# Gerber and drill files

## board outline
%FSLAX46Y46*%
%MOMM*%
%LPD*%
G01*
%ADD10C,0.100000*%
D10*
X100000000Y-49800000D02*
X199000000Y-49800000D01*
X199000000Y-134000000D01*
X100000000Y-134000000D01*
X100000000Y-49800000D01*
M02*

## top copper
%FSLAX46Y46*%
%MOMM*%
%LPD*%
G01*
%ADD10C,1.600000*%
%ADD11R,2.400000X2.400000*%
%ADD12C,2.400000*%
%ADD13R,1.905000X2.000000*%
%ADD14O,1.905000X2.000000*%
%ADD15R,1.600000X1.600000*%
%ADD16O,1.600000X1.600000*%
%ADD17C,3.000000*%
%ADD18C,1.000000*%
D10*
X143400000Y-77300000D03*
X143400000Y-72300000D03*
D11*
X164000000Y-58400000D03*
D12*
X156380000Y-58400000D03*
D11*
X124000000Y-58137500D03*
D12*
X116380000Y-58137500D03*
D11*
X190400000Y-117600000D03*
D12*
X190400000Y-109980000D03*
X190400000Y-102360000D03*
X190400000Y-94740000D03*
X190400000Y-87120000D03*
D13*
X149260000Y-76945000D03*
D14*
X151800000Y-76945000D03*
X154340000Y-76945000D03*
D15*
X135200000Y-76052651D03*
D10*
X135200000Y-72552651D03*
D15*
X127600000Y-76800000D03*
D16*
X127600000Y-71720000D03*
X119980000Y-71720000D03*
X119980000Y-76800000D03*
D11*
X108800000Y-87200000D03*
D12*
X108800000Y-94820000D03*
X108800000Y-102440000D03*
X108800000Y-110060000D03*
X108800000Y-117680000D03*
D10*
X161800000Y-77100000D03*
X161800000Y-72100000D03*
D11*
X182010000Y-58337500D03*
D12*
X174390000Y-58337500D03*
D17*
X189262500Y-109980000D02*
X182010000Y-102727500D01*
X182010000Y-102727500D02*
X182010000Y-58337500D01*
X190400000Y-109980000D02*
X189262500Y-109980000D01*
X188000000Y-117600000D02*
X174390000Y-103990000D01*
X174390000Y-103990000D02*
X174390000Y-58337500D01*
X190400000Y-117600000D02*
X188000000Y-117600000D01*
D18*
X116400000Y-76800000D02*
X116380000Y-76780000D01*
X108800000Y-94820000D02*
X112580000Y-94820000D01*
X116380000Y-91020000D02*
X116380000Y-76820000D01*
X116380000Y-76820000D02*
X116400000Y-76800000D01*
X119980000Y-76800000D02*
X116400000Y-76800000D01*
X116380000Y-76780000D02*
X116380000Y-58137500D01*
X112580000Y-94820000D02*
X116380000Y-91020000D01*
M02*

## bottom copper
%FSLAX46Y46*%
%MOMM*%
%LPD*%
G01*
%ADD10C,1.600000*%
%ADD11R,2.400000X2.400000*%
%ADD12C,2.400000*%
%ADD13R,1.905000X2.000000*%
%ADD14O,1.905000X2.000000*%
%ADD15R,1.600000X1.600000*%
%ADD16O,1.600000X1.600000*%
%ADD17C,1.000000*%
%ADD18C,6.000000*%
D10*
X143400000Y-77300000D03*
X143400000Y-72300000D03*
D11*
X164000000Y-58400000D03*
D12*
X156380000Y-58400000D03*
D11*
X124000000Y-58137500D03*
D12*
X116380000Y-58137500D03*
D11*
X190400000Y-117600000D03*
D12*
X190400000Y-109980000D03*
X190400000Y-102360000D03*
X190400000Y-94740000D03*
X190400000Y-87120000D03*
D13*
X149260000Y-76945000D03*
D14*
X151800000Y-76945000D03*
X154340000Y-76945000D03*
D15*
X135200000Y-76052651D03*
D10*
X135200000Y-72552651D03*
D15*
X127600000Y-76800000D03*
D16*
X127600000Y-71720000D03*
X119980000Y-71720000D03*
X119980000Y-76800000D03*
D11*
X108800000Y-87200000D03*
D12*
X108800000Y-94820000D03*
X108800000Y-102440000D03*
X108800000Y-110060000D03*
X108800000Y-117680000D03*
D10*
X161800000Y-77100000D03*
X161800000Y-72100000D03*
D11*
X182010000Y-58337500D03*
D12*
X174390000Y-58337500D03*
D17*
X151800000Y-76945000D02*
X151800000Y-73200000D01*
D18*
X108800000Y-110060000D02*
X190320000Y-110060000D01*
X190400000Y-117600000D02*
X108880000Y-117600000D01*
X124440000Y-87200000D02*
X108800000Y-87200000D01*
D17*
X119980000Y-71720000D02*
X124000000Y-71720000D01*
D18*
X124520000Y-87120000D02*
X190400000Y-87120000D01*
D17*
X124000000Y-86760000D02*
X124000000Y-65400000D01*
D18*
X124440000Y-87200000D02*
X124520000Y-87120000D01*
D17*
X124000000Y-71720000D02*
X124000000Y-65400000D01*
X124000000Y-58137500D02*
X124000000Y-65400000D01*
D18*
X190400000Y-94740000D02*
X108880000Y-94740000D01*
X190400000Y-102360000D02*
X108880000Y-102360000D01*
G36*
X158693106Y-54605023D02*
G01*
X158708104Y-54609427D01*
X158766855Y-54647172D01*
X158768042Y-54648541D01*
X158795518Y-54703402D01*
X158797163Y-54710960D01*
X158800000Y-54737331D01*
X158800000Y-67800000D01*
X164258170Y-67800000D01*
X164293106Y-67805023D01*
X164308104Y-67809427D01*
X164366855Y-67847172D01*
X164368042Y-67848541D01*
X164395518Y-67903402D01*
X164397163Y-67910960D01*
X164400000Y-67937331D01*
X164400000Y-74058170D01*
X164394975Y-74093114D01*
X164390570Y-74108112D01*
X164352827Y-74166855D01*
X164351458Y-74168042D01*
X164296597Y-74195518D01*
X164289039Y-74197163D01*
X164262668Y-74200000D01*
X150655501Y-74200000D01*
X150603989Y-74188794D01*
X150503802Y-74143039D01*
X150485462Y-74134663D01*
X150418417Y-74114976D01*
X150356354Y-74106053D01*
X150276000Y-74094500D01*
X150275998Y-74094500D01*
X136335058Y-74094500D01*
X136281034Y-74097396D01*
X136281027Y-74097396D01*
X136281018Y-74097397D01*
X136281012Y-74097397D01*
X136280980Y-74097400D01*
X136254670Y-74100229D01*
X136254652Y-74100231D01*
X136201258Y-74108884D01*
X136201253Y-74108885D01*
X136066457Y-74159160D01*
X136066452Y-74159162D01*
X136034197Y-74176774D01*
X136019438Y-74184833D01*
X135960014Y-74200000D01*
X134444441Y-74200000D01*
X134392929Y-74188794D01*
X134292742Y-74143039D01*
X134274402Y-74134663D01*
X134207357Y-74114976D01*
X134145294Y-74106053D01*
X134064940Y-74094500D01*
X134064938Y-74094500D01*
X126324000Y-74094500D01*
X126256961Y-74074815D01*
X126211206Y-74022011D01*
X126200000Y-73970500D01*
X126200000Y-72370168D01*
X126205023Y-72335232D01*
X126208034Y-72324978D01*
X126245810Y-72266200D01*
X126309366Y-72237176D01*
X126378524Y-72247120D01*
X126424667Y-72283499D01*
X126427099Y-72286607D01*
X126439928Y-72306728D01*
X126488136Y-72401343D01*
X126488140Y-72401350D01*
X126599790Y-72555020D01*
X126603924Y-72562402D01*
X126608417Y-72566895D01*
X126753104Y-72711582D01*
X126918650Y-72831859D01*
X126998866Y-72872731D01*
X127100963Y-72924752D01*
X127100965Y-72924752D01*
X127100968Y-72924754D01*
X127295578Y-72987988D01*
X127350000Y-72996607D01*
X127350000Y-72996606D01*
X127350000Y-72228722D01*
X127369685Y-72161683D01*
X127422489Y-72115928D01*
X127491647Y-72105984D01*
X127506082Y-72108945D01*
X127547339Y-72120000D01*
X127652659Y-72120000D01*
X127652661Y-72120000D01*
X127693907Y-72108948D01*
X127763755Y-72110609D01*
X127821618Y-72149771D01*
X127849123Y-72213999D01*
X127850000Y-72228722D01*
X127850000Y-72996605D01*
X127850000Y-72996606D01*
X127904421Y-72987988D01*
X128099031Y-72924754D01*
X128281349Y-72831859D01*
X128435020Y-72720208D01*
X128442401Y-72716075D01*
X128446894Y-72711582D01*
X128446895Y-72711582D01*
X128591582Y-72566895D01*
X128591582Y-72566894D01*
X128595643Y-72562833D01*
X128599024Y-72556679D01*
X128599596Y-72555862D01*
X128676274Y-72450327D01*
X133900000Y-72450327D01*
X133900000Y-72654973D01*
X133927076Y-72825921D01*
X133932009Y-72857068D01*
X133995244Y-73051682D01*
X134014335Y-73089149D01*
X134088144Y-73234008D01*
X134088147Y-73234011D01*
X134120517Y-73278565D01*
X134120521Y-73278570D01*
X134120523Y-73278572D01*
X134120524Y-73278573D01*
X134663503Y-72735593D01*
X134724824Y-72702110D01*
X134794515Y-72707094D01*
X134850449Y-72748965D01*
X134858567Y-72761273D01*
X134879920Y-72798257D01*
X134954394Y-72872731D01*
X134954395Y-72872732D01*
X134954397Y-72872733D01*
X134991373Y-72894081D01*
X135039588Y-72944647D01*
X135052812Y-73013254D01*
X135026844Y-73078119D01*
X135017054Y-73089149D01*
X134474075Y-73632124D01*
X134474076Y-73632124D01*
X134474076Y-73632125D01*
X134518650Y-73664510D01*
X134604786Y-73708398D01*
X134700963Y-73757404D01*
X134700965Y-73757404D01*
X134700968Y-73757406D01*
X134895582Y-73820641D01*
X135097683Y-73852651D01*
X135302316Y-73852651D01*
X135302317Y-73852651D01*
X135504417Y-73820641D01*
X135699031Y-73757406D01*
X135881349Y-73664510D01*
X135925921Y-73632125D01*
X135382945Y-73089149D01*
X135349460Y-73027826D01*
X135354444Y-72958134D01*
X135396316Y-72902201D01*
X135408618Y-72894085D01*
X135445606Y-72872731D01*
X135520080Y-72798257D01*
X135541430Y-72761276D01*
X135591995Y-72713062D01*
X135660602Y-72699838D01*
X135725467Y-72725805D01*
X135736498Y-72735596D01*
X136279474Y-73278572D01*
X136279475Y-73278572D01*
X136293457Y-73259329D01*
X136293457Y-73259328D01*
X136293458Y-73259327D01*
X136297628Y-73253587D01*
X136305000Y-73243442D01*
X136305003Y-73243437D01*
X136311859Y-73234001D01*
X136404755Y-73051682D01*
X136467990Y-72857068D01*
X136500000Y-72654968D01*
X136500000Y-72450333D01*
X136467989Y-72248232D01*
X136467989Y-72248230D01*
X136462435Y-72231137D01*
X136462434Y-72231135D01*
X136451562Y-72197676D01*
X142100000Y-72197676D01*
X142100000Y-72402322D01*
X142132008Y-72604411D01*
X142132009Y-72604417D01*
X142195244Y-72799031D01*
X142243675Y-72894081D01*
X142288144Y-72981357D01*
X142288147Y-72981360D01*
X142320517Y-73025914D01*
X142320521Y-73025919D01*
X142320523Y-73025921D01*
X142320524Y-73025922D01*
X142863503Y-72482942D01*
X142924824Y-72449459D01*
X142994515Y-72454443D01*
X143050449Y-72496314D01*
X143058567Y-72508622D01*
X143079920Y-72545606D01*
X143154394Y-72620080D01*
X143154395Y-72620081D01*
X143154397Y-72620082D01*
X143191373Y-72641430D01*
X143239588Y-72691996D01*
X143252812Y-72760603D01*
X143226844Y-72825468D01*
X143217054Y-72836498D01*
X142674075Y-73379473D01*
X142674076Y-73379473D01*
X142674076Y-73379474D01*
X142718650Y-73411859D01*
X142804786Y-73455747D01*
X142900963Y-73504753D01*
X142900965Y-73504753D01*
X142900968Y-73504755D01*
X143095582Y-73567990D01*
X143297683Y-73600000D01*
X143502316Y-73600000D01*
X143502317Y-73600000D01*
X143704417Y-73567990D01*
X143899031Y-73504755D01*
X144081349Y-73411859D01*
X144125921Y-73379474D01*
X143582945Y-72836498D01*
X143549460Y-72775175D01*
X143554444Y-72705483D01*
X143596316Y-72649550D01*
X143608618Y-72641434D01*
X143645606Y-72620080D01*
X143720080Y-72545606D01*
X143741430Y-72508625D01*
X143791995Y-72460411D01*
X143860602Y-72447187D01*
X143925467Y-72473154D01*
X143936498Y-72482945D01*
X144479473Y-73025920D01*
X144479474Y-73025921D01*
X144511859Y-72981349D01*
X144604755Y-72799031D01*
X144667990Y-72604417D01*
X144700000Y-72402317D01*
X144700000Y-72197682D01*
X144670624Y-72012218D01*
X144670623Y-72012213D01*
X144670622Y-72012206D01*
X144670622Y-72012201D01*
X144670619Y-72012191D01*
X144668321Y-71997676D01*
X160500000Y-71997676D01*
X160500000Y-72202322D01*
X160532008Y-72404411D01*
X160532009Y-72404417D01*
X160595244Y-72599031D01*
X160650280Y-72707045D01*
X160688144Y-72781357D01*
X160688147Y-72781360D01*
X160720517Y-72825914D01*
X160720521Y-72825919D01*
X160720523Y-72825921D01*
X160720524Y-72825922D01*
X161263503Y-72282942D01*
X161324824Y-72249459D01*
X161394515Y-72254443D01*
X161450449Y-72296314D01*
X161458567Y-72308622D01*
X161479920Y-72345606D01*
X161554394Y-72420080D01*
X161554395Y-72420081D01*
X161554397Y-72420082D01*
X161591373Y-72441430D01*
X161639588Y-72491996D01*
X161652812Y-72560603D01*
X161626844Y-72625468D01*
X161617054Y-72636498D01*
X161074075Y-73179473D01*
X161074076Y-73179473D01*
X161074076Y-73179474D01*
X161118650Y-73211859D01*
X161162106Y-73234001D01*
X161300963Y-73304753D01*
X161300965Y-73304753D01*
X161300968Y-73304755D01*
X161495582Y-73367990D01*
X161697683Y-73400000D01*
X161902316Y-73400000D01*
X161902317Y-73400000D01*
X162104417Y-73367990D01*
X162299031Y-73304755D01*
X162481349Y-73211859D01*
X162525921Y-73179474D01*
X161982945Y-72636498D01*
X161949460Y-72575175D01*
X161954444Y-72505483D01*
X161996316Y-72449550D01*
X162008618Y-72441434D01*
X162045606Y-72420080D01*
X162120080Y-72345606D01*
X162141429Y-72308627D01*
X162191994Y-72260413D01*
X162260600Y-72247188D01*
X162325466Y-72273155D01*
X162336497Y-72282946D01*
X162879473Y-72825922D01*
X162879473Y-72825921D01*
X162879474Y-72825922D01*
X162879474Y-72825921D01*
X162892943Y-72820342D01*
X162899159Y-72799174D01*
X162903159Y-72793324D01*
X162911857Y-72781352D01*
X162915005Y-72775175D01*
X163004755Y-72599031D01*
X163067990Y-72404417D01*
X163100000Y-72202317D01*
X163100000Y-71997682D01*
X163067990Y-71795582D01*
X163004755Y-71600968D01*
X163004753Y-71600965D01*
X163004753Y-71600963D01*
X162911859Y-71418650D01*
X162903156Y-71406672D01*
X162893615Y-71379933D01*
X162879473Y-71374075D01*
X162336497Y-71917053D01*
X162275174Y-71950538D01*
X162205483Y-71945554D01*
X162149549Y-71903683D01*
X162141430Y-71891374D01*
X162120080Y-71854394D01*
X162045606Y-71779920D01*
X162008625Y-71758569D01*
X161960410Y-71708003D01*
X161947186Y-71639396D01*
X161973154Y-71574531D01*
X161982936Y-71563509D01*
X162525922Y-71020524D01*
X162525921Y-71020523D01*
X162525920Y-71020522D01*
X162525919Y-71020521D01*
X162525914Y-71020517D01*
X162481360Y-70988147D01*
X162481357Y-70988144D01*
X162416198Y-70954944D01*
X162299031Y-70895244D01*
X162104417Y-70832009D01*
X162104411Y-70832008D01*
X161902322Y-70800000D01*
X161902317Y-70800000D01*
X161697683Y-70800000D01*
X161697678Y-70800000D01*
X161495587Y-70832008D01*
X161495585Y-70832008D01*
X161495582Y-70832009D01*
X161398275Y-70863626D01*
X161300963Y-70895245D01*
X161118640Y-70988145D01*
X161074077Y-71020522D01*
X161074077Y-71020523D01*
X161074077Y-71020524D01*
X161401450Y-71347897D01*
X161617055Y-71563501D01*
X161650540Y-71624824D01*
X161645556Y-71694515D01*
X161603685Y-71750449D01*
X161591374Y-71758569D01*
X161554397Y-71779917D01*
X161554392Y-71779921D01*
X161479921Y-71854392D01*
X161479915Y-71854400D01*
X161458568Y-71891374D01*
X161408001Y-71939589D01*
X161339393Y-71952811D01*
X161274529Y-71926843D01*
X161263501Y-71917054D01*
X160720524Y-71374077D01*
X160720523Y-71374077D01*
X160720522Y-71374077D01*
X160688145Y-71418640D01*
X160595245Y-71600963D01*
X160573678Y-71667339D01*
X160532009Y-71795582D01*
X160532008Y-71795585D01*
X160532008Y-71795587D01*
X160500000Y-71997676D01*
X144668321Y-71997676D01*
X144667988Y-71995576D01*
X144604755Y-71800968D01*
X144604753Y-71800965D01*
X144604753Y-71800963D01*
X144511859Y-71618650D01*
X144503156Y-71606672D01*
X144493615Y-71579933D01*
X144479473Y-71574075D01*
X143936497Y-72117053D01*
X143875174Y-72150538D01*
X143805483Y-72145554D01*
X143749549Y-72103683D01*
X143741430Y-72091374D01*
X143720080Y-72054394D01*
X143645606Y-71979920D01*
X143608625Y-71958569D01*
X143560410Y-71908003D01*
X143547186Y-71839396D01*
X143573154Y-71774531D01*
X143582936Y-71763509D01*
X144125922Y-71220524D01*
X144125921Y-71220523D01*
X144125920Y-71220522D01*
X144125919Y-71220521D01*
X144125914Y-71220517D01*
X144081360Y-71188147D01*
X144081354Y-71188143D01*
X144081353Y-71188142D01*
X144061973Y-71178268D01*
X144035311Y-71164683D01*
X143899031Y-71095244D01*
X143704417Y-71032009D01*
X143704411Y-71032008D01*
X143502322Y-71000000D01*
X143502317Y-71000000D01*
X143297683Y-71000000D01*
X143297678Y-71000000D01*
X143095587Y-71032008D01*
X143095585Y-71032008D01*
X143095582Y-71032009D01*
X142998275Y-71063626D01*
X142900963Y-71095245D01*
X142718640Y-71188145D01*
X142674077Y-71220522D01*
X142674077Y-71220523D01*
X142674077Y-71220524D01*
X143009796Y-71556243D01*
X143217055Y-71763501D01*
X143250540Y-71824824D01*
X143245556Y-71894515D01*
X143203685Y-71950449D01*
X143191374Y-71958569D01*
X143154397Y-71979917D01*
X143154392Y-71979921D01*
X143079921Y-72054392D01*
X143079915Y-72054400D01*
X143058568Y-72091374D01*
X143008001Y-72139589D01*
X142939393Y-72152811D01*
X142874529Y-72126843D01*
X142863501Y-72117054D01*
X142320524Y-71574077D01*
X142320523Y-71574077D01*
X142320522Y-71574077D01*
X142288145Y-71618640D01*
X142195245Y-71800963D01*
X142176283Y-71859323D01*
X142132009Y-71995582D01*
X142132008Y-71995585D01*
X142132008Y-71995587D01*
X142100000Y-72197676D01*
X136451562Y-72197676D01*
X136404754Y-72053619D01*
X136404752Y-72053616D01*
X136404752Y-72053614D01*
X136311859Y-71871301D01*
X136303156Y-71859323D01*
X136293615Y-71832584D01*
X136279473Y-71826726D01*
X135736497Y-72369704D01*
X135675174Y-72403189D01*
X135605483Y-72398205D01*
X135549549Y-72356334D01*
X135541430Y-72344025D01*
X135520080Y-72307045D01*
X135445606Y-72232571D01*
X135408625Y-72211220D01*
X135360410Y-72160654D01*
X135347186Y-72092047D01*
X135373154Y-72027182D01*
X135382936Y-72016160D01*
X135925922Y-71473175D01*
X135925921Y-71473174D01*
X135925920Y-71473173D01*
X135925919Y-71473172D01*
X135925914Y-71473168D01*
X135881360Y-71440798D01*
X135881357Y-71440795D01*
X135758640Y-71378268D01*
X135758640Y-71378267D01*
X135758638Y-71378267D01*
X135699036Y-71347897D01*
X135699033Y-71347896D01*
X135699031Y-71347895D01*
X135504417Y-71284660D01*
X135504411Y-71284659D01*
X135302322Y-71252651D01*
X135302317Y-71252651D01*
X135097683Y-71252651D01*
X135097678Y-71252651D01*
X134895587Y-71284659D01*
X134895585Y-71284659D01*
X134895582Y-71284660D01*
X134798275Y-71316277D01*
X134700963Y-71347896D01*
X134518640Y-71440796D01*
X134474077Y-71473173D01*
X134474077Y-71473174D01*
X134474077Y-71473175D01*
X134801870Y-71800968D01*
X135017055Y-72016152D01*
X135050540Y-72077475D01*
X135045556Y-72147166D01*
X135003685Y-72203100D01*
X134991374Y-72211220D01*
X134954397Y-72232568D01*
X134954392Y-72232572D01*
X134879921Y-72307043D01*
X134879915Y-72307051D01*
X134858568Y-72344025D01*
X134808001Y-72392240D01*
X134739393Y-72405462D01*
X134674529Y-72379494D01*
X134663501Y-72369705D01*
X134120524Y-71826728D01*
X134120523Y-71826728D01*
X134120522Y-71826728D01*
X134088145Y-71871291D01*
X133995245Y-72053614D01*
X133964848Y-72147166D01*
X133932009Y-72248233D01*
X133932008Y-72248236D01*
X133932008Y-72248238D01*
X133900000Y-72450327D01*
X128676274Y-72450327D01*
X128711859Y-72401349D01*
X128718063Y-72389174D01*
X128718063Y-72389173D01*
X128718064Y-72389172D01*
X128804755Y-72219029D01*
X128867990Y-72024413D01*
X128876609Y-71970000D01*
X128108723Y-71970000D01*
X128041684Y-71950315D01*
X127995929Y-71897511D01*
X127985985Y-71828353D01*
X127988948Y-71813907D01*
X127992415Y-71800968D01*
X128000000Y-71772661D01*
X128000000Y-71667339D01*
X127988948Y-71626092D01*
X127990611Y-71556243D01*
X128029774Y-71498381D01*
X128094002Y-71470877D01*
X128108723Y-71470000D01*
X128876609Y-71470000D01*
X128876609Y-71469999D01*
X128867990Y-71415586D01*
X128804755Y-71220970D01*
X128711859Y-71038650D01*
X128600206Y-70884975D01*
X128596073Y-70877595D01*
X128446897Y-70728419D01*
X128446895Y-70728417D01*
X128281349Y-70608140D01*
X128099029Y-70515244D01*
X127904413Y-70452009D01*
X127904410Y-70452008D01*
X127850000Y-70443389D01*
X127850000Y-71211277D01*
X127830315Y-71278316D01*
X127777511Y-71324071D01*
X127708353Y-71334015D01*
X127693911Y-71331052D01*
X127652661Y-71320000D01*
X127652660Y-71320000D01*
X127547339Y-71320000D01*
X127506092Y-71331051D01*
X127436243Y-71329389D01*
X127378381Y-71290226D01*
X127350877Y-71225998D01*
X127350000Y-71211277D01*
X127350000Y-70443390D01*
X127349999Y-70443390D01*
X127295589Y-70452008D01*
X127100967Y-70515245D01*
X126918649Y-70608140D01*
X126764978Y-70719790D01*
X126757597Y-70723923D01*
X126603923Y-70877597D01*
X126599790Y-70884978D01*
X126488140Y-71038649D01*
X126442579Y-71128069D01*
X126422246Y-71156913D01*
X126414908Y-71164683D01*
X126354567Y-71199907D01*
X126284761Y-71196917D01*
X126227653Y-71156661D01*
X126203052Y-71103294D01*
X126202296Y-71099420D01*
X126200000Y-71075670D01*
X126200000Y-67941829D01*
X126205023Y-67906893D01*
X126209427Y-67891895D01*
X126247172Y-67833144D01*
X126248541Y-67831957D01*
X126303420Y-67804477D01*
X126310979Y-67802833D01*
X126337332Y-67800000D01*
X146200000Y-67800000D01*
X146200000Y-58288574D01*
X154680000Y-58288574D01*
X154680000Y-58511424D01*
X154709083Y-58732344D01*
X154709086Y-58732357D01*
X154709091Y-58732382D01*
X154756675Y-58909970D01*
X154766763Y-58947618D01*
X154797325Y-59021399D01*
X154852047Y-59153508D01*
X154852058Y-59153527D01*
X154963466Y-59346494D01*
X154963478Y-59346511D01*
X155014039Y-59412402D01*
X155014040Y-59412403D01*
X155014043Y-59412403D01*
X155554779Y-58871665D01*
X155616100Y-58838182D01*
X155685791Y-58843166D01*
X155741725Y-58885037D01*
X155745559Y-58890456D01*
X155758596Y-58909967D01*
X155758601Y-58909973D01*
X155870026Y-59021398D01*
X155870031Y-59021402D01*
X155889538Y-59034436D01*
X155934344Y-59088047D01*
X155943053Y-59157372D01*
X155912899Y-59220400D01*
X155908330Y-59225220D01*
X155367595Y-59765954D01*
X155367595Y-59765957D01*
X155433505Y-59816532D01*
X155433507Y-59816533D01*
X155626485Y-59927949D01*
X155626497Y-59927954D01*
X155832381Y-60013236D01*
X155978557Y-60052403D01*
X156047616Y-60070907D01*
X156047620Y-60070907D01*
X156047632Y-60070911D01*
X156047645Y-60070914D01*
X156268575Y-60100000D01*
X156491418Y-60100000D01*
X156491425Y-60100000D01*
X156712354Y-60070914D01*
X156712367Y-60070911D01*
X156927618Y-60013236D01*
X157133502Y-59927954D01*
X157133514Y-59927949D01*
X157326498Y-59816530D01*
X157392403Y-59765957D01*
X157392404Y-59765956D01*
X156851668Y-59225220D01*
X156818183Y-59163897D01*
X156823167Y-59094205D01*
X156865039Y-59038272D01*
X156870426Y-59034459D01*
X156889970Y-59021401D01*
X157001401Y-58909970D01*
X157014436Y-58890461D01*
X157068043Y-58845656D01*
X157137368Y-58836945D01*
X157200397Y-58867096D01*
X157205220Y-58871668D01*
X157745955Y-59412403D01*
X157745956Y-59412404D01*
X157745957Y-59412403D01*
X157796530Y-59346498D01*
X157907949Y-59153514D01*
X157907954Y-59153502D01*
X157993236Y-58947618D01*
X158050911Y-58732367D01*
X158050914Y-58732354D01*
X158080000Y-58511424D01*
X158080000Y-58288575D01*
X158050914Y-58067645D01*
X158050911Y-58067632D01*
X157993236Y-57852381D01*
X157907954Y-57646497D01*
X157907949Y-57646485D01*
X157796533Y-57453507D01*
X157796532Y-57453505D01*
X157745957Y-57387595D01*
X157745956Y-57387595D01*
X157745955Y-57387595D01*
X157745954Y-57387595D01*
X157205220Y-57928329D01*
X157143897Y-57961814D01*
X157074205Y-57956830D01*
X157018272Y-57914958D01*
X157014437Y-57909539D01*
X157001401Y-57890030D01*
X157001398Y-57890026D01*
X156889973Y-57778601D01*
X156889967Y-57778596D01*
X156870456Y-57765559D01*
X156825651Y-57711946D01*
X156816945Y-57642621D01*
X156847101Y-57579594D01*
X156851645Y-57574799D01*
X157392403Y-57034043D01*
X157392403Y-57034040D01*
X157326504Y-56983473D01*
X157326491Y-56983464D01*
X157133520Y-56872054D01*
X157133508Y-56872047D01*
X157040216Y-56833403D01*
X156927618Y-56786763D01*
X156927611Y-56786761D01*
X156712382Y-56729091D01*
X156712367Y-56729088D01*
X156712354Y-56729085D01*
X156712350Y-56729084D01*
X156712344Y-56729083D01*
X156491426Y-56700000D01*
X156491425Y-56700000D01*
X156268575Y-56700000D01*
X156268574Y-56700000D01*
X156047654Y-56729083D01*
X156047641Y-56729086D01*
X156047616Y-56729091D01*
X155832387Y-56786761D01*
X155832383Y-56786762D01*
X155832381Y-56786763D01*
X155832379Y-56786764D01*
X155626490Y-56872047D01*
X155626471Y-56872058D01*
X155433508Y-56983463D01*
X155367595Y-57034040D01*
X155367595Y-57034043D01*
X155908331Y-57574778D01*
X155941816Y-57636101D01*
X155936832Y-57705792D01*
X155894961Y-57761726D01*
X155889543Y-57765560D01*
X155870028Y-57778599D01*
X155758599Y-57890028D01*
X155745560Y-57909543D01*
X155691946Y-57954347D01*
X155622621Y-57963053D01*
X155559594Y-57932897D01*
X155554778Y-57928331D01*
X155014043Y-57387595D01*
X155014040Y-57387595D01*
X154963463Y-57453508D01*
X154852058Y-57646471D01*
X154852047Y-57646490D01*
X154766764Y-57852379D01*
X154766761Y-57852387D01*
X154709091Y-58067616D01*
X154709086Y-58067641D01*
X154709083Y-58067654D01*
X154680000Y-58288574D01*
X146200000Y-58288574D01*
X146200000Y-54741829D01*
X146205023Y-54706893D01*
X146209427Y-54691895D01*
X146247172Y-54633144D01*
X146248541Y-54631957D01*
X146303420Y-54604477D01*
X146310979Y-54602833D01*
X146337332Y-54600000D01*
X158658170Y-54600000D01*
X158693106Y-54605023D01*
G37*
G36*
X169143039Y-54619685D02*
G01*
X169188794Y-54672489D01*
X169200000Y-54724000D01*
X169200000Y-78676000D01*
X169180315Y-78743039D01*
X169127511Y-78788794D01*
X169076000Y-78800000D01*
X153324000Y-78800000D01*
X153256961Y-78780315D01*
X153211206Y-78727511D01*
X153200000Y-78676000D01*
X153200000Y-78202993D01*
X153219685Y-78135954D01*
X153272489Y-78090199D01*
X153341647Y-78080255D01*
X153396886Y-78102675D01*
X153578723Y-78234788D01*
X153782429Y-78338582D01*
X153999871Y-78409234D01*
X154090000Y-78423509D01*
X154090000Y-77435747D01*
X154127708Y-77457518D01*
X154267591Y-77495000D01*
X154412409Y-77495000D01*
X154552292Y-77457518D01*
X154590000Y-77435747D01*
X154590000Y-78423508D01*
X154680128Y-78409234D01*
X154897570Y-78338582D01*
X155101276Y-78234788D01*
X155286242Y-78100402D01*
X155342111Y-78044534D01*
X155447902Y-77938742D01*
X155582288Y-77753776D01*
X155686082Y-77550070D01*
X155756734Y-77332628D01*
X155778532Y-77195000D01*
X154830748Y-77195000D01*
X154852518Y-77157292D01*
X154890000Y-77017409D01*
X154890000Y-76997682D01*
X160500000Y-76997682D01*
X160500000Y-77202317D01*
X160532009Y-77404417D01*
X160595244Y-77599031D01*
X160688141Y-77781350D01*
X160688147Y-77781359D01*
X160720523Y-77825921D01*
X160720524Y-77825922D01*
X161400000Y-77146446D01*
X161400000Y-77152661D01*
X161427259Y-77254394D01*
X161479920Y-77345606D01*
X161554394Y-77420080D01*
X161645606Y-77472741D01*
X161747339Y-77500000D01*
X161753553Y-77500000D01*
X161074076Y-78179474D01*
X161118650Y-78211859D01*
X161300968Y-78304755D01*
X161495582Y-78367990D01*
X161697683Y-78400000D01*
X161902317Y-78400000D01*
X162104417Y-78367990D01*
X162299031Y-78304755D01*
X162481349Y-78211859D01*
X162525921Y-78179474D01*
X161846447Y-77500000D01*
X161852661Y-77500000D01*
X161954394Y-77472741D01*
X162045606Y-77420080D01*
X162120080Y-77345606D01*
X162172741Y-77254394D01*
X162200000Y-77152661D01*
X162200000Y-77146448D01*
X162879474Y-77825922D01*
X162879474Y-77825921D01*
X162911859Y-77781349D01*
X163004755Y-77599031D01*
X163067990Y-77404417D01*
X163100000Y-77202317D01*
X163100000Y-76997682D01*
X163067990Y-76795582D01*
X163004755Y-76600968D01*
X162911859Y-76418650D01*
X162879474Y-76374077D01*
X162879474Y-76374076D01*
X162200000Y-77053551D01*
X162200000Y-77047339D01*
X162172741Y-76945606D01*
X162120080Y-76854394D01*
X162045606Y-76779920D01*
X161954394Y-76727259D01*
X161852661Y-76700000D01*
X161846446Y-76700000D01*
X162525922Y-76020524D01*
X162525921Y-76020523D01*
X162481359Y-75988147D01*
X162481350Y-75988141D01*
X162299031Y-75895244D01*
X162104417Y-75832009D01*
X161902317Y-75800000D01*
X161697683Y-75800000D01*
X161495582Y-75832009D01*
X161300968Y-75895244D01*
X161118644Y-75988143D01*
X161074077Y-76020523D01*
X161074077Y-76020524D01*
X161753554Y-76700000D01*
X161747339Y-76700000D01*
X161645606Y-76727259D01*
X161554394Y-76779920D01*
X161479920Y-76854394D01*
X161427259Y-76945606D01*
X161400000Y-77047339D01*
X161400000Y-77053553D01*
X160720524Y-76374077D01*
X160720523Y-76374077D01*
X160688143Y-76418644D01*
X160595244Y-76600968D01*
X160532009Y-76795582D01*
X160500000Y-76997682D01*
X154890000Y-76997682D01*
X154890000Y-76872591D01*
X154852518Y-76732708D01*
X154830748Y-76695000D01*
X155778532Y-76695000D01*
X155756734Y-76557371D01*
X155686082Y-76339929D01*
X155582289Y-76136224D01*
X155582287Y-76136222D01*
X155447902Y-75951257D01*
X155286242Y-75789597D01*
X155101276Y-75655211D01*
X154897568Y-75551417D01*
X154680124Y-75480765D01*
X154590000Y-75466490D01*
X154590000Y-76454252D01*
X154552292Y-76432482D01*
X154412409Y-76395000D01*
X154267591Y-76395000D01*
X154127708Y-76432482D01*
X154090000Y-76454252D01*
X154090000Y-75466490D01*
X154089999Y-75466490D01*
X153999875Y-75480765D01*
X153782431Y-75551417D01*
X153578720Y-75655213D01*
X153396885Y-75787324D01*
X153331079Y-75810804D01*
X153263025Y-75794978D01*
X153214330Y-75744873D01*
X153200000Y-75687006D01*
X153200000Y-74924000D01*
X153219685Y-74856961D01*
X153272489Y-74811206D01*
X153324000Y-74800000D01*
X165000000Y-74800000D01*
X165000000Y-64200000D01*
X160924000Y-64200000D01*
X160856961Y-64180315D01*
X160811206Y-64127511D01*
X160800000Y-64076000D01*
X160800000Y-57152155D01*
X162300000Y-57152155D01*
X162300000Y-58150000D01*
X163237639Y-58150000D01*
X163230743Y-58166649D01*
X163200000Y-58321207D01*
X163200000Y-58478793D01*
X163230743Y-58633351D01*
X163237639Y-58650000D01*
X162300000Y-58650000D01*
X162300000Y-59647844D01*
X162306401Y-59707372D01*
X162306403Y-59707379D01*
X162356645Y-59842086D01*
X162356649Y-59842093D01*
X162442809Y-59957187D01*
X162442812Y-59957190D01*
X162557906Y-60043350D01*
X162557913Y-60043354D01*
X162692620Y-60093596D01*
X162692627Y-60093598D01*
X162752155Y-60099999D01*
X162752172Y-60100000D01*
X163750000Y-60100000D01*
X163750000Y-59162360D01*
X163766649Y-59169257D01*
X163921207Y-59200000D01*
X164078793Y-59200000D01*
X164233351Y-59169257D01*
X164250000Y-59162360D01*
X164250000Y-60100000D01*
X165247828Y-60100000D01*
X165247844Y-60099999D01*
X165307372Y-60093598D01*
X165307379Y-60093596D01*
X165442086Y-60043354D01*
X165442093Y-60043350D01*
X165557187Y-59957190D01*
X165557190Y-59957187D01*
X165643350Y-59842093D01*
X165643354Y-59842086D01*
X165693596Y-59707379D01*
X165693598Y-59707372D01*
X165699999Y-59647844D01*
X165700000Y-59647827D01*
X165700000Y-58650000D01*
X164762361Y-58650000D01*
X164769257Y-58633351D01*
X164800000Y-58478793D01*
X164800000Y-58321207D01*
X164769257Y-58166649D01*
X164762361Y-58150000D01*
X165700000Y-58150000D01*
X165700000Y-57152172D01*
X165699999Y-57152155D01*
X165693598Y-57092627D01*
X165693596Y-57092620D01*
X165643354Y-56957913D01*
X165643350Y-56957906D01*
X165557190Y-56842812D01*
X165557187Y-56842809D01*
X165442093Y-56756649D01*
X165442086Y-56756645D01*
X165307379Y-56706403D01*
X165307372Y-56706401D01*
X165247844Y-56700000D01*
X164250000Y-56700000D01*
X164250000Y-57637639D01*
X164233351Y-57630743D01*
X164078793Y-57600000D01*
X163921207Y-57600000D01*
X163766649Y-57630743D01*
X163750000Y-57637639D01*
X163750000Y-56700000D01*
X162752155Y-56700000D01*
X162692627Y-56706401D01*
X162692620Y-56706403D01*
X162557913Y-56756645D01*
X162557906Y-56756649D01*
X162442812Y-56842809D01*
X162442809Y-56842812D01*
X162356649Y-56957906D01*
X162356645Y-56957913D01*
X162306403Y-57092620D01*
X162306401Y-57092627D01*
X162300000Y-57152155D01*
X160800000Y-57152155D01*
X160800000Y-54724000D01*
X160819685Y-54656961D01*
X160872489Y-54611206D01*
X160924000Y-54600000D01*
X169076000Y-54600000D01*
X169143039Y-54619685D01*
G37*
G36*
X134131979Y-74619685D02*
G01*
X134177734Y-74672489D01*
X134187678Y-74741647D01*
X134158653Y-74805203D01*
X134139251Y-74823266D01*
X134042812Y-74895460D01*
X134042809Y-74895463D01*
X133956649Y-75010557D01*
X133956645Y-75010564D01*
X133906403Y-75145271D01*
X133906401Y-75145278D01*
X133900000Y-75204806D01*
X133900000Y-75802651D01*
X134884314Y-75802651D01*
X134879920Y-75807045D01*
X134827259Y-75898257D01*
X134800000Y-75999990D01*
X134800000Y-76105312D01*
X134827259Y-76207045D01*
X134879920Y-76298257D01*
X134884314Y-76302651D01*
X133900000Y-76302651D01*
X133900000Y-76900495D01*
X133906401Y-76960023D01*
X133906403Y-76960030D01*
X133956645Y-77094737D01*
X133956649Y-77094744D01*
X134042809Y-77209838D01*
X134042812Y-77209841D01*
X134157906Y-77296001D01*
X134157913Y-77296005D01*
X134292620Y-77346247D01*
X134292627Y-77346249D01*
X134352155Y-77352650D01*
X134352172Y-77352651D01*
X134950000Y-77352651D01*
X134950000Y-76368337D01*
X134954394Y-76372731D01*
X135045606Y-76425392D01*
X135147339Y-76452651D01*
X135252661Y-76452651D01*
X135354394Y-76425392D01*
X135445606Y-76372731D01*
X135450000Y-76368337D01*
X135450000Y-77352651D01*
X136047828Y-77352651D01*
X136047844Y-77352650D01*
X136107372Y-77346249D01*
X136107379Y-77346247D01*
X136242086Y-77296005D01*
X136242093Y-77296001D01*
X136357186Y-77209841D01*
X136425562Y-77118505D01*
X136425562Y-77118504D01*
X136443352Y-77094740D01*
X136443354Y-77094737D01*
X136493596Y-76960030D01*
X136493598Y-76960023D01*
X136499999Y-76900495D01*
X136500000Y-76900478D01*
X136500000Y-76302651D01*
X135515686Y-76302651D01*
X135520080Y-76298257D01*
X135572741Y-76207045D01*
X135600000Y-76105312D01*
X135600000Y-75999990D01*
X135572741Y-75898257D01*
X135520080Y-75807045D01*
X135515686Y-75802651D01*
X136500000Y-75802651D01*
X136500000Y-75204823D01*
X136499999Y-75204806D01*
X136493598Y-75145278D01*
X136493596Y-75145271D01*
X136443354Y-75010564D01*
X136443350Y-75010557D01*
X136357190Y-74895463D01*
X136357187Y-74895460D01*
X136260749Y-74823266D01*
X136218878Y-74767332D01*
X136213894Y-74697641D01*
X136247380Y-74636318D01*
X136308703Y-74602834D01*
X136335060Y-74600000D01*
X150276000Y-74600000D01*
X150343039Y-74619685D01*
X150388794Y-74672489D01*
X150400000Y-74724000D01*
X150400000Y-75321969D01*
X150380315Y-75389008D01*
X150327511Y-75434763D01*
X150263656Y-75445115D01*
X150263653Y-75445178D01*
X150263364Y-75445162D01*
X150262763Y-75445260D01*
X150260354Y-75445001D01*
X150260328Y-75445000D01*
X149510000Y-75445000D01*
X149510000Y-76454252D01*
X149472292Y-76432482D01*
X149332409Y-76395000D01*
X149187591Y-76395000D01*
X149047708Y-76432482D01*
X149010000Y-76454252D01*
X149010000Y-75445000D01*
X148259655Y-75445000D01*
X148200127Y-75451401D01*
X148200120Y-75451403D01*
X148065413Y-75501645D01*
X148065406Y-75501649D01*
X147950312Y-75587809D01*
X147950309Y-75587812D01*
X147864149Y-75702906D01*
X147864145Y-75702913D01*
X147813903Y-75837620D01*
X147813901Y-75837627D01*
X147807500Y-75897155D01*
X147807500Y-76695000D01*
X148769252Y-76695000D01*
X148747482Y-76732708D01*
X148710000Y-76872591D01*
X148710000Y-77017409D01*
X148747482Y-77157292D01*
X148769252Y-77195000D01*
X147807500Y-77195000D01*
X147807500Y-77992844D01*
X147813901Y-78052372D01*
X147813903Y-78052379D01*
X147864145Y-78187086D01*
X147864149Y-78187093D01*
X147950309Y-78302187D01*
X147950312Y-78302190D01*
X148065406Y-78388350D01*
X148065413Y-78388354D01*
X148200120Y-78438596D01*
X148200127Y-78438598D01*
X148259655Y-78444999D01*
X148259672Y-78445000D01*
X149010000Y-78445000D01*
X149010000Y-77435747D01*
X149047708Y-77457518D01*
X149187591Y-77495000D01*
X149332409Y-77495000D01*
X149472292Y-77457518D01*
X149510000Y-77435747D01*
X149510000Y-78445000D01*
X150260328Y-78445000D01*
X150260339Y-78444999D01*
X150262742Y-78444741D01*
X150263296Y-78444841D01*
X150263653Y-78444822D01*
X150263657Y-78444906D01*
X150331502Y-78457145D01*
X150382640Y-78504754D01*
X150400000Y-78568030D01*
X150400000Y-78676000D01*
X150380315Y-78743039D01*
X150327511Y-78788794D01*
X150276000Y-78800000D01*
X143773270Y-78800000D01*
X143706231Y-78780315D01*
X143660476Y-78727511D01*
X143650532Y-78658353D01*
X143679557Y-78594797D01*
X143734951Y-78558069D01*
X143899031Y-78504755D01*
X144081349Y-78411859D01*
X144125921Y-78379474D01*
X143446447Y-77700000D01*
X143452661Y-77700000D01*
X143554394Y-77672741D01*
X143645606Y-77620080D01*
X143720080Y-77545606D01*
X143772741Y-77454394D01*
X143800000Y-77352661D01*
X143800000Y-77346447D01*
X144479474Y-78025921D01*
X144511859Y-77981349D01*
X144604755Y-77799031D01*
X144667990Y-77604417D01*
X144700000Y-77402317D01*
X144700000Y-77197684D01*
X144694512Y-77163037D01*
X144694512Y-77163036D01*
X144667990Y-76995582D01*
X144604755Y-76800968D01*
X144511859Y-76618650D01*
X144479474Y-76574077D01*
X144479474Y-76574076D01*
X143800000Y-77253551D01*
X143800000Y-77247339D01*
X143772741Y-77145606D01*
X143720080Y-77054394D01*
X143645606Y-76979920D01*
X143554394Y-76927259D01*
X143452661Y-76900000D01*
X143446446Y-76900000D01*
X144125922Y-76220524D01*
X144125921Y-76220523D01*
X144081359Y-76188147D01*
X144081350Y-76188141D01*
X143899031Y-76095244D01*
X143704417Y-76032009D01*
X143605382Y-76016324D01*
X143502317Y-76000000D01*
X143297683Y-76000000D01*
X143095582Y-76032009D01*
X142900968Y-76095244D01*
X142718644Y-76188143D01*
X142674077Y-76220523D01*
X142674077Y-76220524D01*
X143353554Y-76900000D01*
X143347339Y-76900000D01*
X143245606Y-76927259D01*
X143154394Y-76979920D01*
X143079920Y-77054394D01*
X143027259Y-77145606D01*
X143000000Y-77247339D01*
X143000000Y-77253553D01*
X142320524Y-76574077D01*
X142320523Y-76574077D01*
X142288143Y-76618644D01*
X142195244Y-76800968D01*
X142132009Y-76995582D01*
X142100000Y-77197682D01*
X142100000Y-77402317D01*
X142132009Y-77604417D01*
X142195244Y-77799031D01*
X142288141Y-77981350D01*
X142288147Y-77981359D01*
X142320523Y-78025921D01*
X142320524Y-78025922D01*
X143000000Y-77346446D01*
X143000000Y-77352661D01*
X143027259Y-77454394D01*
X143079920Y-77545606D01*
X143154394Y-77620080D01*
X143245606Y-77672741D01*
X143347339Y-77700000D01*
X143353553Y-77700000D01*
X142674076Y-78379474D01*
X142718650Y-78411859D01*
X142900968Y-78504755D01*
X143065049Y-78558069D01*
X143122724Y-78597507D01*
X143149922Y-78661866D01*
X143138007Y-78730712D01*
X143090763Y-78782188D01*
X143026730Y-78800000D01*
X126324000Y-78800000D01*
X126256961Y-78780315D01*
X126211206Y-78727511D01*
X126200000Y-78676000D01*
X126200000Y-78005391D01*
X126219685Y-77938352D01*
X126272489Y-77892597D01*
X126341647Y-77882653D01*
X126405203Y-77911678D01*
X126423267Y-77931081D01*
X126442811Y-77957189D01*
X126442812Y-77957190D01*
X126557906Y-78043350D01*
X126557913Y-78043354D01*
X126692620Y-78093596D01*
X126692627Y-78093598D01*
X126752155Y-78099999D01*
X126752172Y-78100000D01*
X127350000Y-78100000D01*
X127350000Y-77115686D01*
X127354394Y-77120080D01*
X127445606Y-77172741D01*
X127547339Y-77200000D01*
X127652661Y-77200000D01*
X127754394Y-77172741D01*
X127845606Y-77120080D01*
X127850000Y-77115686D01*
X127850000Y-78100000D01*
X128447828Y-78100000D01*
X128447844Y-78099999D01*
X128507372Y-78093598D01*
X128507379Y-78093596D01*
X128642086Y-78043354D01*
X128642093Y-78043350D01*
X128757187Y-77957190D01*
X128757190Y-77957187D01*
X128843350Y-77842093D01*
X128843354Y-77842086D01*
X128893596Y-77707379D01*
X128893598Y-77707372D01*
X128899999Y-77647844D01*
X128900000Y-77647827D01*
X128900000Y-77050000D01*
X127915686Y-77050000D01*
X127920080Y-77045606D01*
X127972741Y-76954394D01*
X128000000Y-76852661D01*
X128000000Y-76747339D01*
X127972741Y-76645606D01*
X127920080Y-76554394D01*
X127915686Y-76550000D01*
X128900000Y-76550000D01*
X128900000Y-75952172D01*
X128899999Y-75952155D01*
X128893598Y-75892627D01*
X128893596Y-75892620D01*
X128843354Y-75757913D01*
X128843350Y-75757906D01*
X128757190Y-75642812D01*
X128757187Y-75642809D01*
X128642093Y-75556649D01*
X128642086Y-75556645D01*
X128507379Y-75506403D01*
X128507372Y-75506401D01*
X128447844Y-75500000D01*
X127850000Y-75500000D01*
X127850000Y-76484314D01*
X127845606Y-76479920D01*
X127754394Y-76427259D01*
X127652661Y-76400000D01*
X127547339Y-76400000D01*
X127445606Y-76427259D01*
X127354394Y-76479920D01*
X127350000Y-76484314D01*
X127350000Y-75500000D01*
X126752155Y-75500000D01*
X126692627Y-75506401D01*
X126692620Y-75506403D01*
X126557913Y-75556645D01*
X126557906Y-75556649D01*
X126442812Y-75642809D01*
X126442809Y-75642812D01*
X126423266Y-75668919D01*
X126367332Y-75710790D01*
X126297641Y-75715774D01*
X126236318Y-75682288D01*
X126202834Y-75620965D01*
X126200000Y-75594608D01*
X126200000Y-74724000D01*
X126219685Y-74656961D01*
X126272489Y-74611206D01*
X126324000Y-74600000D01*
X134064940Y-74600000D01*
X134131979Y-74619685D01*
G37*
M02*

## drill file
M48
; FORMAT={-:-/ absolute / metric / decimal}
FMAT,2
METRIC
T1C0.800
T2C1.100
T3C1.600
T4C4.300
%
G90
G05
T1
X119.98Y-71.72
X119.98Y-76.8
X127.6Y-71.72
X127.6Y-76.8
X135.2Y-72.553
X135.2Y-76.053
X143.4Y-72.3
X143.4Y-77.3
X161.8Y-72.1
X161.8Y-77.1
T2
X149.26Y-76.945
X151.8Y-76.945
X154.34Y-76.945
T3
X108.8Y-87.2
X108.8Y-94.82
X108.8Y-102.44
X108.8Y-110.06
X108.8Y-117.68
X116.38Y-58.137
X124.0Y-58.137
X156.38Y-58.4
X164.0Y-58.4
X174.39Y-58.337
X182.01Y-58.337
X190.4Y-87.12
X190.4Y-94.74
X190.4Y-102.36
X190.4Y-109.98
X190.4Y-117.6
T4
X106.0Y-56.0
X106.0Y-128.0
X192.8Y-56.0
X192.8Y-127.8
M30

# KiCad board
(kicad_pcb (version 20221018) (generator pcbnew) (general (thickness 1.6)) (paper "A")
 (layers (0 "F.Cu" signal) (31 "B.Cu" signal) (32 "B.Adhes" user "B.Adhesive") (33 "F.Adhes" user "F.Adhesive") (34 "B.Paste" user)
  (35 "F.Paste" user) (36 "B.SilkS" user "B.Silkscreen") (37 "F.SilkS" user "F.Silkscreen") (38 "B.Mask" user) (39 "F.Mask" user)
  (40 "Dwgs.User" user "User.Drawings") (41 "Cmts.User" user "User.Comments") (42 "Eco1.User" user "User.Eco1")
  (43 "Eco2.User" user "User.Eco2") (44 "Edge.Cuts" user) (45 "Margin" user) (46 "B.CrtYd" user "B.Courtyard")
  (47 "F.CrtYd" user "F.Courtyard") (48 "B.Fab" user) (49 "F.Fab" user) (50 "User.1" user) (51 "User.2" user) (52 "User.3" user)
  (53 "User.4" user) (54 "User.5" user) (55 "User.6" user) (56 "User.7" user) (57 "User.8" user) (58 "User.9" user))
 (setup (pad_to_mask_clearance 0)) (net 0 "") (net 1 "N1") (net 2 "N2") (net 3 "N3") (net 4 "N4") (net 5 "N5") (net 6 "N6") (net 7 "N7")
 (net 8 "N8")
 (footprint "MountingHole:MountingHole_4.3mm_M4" (layer "F.Cu") (at 106 56)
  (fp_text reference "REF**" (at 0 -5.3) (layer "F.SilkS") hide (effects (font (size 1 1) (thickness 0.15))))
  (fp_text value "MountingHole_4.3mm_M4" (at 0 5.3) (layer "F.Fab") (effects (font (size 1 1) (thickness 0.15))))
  (pad "" np_thru_hole circle (at 0 0) (size 4.3 4.3) (drill 4.3) (layers "*.Cu" "*.Mask")))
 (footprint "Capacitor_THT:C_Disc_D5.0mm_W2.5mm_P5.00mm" (layer "F.Cu") (at 143.4 77.3 90)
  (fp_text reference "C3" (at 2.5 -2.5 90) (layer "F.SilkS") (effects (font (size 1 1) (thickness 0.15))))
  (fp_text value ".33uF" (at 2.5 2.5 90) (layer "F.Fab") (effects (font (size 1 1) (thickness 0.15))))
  (pad "1" thru_hole circle (at 0 0 90) (size 1.6 1.6) (drill 0.8) (layers "*.Cu" "*.Mask") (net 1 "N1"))
  (pad "2" thru_hole circle (at 5 0 90) (size 1.6 1.6) (drill 0.8) (layers "*.Cu" "*.Mask") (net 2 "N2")))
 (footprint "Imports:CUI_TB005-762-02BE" (layer "F.Cu") (at 164 58.4 180)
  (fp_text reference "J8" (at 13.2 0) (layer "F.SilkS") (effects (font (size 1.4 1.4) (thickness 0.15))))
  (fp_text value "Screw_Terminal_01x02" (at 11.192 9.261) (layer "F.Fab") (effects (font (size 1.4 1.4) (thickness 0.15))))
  (pad "1" thru_hole rect (at 0 0 180) (size 2.4 2.4) (drill 1.6) (layers "*.Cu" "*.Mask") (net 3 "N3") (solder_mask_margin 0.102))
  (pad "2" thru_hole circle (at 7.62 0 180) (size 2.4 2.4) (drill 1.6) (layers "*.Cu" "*.Mask") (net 2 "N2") (solder_mask_margin 0.102)))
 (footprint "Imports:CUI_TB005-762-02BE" (layer "F.Cu") (at 124 58.1375 180)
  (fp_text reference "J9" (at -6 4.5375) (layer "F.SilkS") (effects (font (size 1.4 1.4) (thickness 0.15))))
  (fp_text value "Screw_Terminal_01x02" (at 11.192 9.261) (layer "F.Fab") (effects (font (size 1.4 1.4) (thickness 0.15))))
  (pad "1" thru_hole rect (at 0 0 180) (size 2.4 2.4) (drill 1.6) (layers "*.Cu" "*.Mask") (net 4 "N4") (solder_mask_margin 0.102))
  (pad "2" thru_hole circle (at 7.62 0 180) (size 2.4 2.4) (drill 1.6) (layers "*.Cu" "*.Mask") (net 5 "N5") (solder_mask_margin 0.102)))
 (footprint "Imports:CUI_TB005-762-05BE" (layer "F.Cu") (at 190.4 117.6 90)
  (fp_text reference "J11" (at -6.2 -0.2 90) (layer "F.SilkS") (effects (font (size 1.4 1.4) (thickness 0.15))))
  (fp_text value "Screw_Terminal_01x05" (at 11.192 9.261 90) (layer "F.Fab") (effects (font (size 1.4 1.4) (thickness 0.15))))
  (pad "1" thru_hole rect (at 0 0 90) (size 2.4 2.4) (drill 1.6) (layers "*.Cu" "*.Mask") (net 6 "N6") (solder_mask_margin 0.102))
  (pad "2" thru_hole circle (at 7.62 0 90) (size 2.4 2.4) (drill 1.6) (layers "*.Cu" "*.Mask") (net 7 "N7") (solder_mask_margin 0.102))
  (pad "3" thru_hole circle (at 15.24 0 90) (size 2.4 2.4) (drill 1.6) (layers "*.Cu" "*.Mask") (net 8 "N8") (solder_mask_margin 0.102))
  (pad "4" thru_hole circle (at 22.86 0 90) (size 2.4 2.4) (drill 1.6) (layers "*.Cu" "*.Mask") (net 5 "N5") (solder_mask_margin 0.102))
  (pad "5" thru_hole circle (at 30.48 0 90) (size 2.4 2.4) (drill 1.6) (layers "*.Cu" "*.Mask") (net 4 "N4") (solder_mask_margin 0.102)))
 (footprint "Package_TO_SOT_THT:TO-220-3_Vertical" (layer "F.Cu") (at 149.26 76.945)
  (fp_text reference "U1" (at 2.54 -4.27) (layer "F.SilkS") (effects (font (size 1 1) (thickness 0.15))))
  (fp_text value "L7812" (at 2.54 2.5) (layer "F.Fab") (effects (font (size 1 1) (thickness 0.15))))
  (pad "1" thru_hole rect (at 0 0) (size 1.905 2) (drill 1.1) (layers "*.Cu" "*.Mask") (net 1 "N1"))
  (pad "2" thru_hole oval (at 2.54 0) (size 1.905 2) (drill 1.1) (layers "*.Cu" "*.Mask") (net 2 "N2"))
  (pad "3" thru_hole oval (at 5.08 0) (size 1.905 2) (drill 1.1) (layers "*.Cu" "*.Mask") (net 3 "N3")))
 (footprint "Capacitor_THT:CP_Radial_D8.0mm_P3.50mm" (layer "F.Cu") (at 135.2 76.052651 90)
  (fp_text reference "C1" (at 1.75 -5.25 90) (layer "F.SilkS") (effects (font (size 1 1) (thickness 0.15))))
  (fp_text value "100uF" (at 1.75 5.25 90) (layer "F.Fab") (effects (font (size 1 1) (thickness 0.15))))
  (pad "1" thru_hole rect (at 0 0 90) (size 1.6 1.6) (drill 0.8) (layers "*.Cu" "*.Mask") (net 1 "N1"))
  (pad "2" thru_hole circle (at 3.5 0 90) (size 1.6 1.6) (drill 0.8) (layers "*.Cu" "*.Mask") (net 2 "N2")))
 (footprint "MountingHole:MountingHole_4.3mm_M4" (layer "F.Cu") (at 106 128)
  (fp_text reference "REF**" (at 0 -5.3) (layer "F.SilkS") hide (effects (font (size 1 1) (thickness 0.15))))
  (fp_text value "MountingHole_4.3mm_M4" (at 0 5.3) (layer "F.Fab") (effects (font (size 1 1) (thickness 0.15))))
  (pad "" np_thru_hole circle (at 0 0) (size 4.3 4.3) (drill 4.3) (layers "*.Cu" "*.Mask")))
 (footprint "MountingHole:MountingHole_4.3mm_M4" (layer "F.Cu") (at 192.8 56)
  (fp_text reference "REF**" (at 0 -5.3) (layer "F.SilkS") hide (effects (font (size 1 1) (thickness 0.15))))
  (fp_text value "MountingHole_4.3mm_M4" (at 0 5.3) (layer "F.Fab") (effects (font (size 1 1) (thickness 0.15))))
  (pad "" np_thru_hole circle (at 0 0) (size 4.3 4.3) (drill 4.3) (layers "*.Cu" "*.Mask")))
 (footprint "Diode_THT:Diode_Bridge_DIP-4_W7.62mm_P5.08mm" (layer "F.Cu") (at 127.6 76.8 180)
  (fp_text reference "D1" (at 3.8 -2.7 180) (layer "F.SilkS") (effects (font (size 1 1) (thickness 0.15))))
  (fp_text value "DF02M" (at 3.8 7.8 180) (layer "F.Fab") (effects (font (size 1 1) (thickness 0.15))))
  (pad "1" thru_hole rect (at 0 0 180) (size 1.6 1.6) (drill 0.8) (layers "*.Cu" "*.Mask") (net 1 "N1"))
  (pad "2" thru_hole oval (at 0 5.08 180) (size 1.6 1.6) (drill 0.8) (layers "*.Cu" "*.Mask") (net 2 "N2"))
  (pad "3" thru_hole oval (at 7.62 5.08 180) (size 1.6 1.6) (drill 0.8) (layers "*.Cu" "*.Mask") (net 4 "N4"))
  (pad "4" thru_hole oval (at 7.62 0 180) (size 1.6 1.6) (drill 0.8) (layers "*.Cu" "*.Mask") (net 5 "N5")))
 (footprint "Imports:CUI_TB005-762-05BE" (layer "F.Cu") (at 108.8 87.2 -90)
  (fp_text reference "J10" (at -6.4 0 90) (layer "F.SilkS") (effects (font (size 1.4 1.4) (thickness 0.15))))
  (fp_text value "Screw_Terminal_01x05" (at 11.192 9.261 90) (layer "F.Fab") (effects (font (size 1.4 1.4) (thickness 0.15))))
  (pad "1" thru_hole rect (at 0 0 270) (size 2.4 2.4) (drill 1.6) (layers "*.Cu" "*.Mask") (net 4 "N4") (solder_mask_margin 0.102))
  (pad "2" thru_hole circle (at 7.62 0 270) (size 2.4 2.4) (drill 1.6) (layers "*.Cu" "*.Mask") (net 5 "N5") (solder_mask_margin 0.102))
  (pad "3" thru_hole circle (at 15.24 0 270) (size 2.4 2.4) (drill 1.6) (layers "*.Cu" "*.Mask") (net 8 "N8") (solder_mask_margin 0.102))
  (pad "4" thru_hole circle (at 22.86 0 270) (size 2.4 2.4) (drill 1.6) (layers "*.Cu" "*.Mask") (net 7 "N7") (solder_mask_margin 0.102))
  (pad "5" thru_hole circle (at 30.48 0 270) (size 2.4 2.4) (drill 1.6) (layers "*.Cu" "*.Mask") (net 6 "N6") (solder_mask_margin 0.102)))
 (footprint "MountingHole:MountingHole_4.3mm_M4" (layer "F.Cu") (at 192.8 127.8)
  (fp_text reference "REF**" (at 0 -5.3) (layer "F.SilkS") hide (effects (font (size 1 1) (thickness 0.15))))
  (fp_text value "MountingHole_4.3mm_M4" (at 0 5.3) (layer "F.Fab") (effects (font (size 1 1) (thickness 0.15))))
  (pad "" np_thru_hole circle (at 0 0) (size 4.3 4.3) (drill 4.3) (layers "*.Cu" "*.Mask")))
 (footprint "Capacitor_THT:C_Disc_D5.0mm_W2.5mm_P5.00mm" (layer "F.Cu") (at 161.8 77.1 90)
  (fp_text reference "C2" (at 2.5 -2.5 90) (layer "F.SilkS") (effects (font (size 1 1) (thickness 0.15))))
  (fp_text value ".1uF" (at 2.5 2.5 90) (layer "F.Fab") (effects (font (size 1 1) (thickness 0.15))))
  (pad "1" thru_hole circle (at 0 0 90) (size 1.6 1.6) (drill 0.8) (layers "*.Cu" "*.Mask") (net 3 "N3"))
  (pad "2" thru_hole circle (at 5 0 90) (size 1.6 1.6) (drill 0.8) (layers "*.Cu" "*.Mask") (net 2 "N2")))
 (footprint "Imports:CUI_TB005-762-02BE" (layer "F.Cu") (at 182.01 58.3375 180)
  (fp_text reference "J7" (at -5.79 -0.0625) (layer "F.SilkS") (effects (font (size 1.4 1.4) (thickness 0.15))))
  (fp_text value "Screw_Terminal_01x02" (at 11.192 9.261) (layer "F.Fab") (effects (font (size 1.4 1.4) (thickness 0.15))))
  (pad "1" thru_hole rect (at 0 0 180) (size 2.4 2.4) (drill 1.6) (layers "*.Cu" "*.Mask") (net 7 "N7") (solder_mask_margin 0.102))
  (pad "2" thru_hole circle (at 7.62 0 180) (size 2.4 2.4) (drill 1.6) (layers "*.Cu" "*.Mask") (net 6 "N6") (solder_mask_margin 0.102)))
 (gr_rect (start 100 49.8) (end 199 134) (stroke (width 0.1) (type default)) (fill none) (layer "Edge.Cuts"))
 (segment (start 151.8 76.945) (end 151.8 73.2) (width 1) (layer "B.Cu") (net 2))
 (segment (start 189.2625 109.98) (end 182.01 102.7275) (width 3) (layer "F.Cu") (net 7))
 (segment (start 182.01 102.7275) (end 182.01 58.3375) (width 3) (layer "F.Cu") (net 7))
 (segment (start 190.4 109.98) (end 189.2625 109.98) (width 3) (layer "F.Cu") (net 7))
 (segment (start 108.8 110.06) (end 190.32 110.06) (width 6) (layer "B.Cu") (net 7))
 (segment (start 188 117.6) (end 174.39 103.99) (width 3) (layer "F.Cu") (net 6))
 (segment (start 174.39 103.99) (end 174.39 58.3375) (width 3) (layer "F.Cu") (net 6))
 (segment (start 190.4 117.6) (end 188 117.6) (width 3) (layer "F.Cu") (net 6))
 (segment (start 190.4 117.6) (end 108.88 117.6) (width 6) (layer "B.Cu") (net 6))
 (segment (start 124.44 87.2) (end 108.8 87.2) (width 6) (layer "B.Cu") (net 4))
 (segment (start 119.98 71.72) (end 124 71.72) (width 1) (layer "B.Cu") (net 4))
 (segment (start 124.52 87.12) (end 190.4 87.12) (width 6) (layer "B.Cu") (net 4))
 (segment (start 124 86.76) (end 124 65.4) (width 1) (layer "B.Cu") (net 4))
 (segment (start 124.44 87.2) (end 124.52 87.12) (width 6) (layer "B.Cu") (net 4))
 (segment (start 124 71.72) (end 124 65.4) (width 1) (layer "B.Cu") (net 4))
 (segment (start 124 58.1375) (end 124 65.4) (width 1) (layer "B.Cu") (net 4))
 (segment (start 116.4 76.8) (end 116.38 76.78) (width 1) (layer "F.Cu") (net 5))
 (segment (start 108.8 94.82) (end 112.58 94.82) (width 1) (layer "F.Cu") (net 5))
 (segment (start 116.38 91.02) (end 116.38 76.82) (width 1) (layer "F.Cu") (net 5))
 (segment (start 116.38 76.82) (end 116.4 76.8) (width 1) (layer "F.Cu") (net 5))
 (segment (start 119.98 76.8) (end 116.4 76.8) (width 1) (layer "F.Cu") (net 5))
 (segment (start 116.38 76.78) (end 116.38 58.1375) (width 1) (layer "F.Cu") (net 5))
 (segment (start 112.58 94.82) (end 116.38 91.02) (width 1) (layer "F.Cu") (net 5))
 (segment (start 190.4 94.74) (end 108.88 94.74) (width 6) (layer "B.Cu") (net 5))
 (segment (start 190.4 102.36) (end 108.88 102.36) (width 6) (layer "B.Cu") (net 8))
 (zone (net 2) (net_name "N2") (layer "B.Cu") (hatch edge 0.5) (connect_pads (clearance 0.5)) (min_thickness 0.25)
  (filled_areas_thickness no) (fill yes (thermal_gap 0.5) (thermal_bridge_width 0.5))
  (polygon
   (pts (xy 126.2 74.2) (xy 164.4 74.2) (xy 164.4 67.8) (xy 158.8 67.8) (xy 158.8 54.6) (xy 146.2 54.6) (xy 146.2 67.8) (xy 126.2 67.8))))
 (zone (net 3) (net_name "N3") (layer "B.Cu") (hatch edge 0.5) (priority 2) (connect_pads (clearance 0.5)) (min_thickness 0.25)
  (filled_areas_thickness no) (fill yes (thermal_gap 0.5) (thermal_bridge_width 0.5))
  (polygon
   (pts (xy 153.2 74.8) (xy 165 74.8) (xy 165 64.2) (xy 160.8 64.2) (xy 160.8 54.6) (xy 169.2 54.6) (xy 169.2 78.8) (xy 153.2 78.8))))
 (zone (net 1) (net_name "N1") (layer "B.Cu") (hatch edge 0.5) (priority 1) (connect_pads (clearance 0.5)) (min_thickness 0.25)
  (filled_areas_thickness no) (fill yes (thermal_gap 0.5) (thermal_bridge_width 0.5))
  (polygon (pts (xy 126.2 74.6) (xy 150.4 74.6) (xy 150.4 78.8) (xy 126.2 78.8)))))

